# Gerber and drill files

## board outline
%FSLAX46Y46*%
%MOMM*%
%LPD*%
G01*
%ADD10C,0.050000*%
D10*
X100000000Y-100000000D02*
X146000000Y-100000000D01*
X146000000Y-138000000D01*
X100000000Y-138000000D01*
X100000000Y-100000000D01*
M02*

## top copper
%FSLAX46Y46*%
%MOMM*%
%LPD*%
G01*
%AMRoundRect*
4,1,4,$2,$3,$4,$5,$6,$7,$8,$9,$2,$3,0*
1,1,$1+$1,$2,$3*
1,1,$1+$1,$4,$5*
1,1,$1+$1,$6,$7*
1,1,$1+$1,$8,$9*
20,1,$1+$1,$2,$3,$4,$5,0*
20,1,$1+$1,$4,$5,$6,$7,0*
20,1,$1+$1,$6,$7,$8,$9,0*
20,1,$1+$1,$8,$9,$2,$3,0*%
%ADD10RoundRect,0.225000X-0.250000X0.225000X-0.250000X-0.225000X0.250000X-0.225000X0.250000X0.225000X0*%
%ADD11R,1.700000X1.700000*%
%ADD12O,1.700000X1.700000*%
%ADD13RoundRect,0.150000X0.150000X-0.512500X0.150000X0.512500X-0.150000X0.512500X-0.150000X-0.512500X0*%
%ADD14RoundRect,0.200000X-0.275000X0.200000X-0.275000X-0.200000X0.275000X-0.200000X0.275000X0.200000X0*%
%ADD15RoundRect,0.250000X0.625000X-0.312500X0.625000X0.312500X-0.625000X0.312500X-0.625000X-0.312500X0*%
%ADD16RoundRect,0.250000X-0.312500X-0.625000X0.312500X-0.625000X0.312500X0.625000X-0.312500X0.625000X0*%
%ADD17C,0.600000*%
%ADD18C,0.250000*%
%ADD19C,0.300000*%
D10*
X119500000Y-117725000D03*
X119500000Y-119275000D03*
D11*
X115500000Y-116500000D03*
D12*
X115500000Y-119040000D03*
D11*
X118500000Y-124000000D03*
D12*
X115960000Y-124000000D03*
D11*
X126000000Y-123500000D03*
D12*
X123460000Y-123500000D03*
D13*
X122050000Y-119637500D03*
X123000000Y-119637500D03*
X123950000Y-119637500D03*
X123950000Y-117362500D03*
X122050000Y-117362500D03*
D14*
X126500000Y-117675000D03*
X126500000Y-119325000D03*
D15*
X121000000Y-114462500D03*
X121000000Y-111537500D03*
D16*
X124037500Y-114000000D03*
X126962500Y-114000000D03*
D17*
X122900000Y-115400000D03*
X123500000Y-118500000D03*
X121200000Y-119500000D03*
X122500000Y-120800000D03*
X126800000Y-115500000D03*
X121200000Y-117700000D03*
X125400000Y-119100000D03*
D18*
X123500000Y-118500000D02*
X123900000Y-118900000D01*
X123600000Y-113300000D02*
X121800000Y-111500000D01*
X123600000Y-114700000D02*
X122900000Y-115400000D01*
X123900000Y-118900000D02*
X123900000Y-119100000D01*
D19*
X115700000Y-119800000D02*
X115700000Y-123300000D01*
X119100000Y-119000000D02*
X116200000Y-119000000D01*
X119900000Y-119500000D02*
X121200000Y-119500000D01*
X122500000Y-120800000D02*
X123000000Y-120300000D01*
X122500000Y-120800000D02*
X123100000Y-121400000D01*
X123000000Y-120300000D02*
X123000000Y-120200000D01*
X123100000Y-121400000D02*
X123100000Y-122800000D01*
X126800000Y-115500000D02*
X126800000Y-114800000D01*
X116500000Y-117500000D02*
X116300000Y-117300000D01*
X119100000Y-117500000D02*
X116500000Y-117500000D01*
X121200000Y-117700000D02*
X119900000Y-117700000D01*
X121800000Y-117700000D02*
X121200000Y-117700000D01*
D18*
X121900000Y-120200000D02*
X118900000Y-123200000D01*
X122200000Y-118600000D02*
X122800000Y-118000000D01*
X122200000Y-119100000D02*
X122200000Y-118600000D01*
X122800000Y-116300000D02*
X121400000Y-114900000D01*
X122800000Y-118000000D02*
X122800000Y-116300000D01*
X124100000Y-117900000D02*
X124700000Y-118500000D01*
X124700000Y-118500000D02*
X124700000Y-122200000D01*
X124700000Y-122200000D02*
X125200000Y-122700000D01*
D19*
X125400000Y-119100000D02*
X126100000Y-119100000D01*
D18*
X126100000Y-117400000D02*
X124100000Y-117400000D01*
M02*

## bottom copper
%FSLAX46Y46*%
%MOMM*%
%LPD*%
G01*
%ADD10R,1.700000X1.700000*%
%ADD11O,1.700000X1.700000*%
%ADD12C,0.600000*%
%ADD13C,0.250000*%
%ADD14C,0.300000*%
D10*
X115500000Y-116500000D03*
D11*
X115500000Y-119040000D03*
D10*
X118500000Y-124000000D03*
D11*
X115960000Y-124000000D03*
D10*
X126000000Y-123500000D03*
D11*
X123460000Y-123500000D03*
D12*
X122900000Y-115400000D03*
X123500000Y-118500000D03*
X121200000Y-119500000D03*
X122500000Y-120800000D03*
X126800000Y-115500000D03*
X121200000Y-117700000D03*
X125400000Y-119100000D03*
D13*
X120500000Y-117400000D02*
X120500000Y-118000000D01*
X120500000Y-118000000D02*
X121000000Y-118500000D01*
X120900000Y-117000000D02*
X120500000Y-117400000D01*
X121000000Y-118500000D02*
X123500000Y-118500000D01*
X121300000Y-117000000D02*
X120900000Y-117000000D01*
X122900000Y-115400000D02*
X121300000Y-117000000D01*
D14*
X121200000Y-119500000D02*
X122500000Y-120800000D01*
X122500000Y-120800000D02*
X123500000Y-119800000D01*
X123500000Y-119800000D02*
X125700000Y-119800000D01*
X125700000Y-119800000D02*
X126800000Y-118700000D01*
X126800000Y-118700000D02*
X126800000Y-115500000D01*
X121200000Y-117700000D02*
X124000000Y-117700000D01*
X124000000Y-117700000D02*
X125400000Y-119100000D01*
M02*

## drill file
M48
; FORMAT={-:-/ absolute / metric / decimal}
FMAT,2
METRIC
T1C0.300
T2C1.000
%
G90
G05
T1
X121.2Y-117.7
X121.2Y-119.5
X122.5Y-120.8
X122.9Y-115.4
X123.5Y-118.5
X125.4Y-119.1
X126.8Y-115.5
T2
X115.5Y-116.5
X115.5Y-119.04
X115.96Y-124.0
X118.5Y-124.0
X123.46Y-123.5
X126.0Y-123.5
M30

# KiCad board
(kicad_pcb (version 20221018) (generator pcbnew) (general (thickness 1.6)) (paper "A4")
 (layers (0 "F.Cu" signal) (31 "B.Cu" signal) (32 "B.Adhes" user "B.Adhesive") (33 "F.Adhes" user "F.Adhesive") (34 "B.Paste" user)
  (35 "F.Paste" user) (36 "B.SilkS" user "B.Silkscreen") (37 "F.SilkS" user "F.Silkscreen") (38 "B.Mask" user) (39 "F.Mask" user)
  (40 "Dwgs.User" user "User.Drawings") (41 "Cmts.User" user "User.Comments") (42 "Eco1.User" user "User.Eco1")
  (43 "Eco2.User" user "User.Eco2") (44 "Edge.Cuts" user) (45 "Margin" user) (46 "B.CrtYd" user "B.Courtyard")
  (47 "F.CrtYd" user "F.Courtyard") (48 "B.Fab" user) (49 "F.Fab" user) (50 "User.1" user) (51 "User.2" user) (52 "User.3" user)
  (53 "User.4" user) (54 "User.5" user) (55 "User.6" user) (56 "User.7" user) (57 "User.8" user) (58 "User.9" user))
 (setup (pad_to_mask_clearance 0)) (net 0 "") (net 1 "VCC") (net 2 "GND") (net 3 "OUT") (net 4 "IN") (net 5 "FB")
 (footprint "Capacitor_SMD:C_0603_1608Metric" (layer "F.Cu") (at 119.5 118.5 -90)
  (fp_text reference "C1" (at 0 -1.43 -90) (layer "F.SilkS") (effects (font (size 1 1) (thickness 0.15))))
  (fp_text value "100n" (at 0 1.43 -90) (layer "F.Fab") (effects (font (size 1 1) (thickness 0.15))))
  (pad "1" smd roundrect (at -0.775 0 270) (size 0.9 0.95) (layers "F.Cu" "F.Paste" "F.Mask") (roundrect_rratio 0.25) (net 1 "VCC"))
  (pad "2" smd roundrect (at 0.775 0 270) (size 0.9 0.95) (layers "F.Cu" "F.Paste" "F.Mask") (roundrect_rratio 0.25) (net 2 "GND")))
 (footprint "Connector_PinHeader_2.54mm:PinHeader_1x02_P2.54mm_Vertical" (layer "F.Cu") (at 115.5 116.5)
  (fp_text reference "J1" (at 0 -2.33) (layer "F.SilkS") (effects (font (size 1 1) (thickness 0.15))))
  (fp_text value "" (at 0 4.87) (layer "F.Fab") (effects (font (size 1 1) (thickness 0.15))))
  (pad "1" thru_hole rect (at 0 0) (size 1.7 1.7) (drill 1) (layers "*.Cu" "*.Mask") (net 1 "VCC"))
  (pad "2" thru_hole oval (at 0 2.54) (size 1.7 1.7) (drill 1) (layers "*.Cu" "*.Mask") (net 2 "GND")))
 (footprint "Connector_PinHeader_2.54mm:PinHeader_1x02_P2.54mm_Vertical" (layer "F.Cu") (at 118.5 124 -90)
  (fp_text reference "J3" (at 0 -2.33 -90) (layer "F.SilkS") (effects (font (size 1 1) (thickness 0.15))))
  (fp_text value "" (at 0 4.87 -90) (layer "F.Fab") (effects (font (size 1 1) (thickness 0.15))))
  (pad "1" thru_hole rect (at 0 0 270) (size 1.7 1.7) (drill 1) (layers "*.Cu" "*.Mask") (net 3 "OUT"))
  (pad "2" thru_hole oval (at 0 2.54 270) (size 1.7 1.7) (drill 1) (layers "*.Cu" "*.Mask") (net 2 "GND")))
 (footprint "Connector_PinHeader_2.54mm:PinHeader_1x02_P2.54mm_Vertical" (layer "F.Cu") (at 126 123.5 -90)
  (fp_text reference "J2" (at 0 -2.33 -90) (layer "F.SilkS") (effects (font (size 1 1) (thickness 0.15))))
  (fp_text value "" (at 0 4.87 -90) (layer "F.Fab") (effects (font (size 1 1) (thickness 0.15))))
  (pad "1" thru_hole rect (at 0 0 270) (size 1.7 1.7) (drill 1) (layers "*.Cu" "*.Mask") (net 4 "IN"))
  (pad "2" thru_hole oval (at 0 2.54 270) (size 1.7 1.7) (drill 1) (layers "*.Cu" "*.Mask") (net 2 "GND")))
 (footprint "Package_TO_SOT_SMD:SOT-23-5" (layer "F.Cu") (at 123 118.5 90)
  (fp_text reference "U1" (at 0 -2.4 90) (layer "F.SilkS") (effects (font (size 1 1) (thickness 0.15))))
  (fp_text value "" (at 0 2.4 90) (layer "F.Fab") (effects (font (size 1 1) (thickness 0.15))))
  (pad "1" smd roundrect (at -1.1375 -0.95 90) (size 1.325 0.6) (layers "F.Cu" "F.Paste" "F.Mask") (roundrect_rratio 0.25) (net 3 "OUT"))
  (pad "2" smd roundrect (at -1.1375 0 90) (size 1.325 0.6) (layers "F.Cu" "F.Paste" "F.Mask") (roundrect_rratio 0.25) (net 2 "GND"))
  (pad "3" smd roundrect (at -1.1375 0.95 90) (size 1.325 0.6) (layers "F.Cu" "F.Paste" "F.Mask") (roundrect_rratio 0.25) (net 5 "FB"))
  (pad "4" smd roundrect (at 1.1375 0.95 90) (size 1.325 0.6) (layers "F.Cu" "F.Paste" "F.Mask") (roundrect_rratio 0.25) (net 4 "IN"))
  (pad "5" smd roundrect (at 1.1375 -0.95 90) (size 1.325 0.6) (layers "F.Cu" "F.Paste" "F.Mask") (roundrect_rratio 0.25) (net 1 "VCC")))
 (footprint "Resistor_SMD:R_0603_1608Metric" (layer "F.Cu") (at 126.5 118.5 -90)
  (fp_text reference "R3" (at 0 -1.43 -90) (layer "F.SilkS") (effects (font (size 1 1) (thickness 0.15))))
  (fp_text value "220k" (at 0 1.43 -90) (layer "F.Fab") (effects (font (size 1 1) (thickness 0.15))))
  (pad "1" smd roundrect (at -0.825 0 270) (size 0.8 0.95) (layers "F.Cu" "F.Paste" "F.Mask") (roundrect_rratio 0.25) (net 4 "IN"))
  (pad "2" smd roundrect (at 0.825 0 270) (size 0.8 0.95) (layers "F.Cu" "F.Paste" "F.Mask") (roundrect_rratio 0.25) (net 1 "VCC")))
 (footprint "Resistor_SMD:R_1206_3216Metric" (layer "F.Cu") (at 121 113 90)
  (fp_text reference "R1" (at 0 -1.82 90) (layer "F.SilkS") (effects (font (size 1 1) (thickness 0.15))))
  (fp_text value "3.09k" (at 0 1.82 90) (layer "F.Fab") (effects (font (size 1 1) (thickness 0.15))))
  (pad "1" smd roundrect (at -1.4625 0 90) (size 1.125 1.75) (layers "F.Cu" "F.Paste" "F.Mask") (roundrect_rratio 0.222222) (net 3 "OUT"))
  (pad "2" smd roundrect (at 1.4625 0 90) (size 1.125 1.75) (layers "F.Cu" "F.Paste" "F.Mask") (roundrect_rratio 0.222222) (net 5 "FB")))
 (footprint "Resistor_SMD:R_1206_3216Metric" (layer "F.Cu") (at 125.5 114)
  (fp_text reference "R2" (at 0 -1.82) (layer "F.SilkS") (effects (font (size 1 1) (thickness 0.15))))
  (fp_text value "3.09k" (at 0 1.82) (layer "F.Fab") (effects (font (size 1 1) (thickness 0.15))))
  (pad "1" smd roundrect (at -1.4625 0) (size 1.125 1.75) (layers "F.Cu" "F.Paste" "F.Mask") (roundrect_rratio 0.222222) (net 5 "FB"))
  (pad "2" smd roundrect (at 1.4625 0) (size 1.125 1.75) (layers "F.Cu" "F.Paste" "F.Mask") (roundrect_rratio 0.222222) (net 2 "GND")))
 (gr_rect (start 100 100) (end 146 138) (stroke (width 0.05) (type default)) (fill none) (layer "Edge.Cuts"))
 (segment (start 123.5 118.5) (end 123.9 118.9) (width 0.25) (layer "F.Cu") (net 5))
 (segment (start 123.6 113.3) (end 121.8 111.5) (width 0.25) (layer "F.Cu") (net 5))
 (segment (start 123.6 114.7) (end 122.9 115.4) (width 0.25) (layer "F.Cu") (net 5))
 (segment (start 123.9 118.9) (end 123.9 119.1) (width 0.25) (layer "F.Cu") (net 5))
 (via (at 122.9 115.4) (size 0.6) (drill 0.3) (layers "F.Cu" "B.Cu") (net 5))
 (via (at 123.5 118.5) (size 0.6) (drill 0.3) (layers "F.Cu" "B.Cu") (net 5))
 (segment (start 115.7 119.8) (end 115.7 123.3) (width 0.3) (layer "F.Cu") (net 2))
 (segment (start 119.1 119) (end 116.2 119) (width 0.3) (layer "F.Cu") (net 2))
 (segment (start 119.9 119.5) (end 121.2 119.5) (width 0.3) (layer "F.Cu") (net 2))
 (segment (start 120.5 117.4) (end 120.5 118) (width 0.25) (layer "B.Cu") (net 5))
 (segment (start 120.5 118) (end 121 118.5) (width 0.25) (layer "B.Cu") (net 5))
 (segment (start 120.9 117) (end 120.5 117.4) (width 0.25) (layer "B.Cu") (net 5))
 (segment (start 121 118.5) (end 123.5 118.5) (width 0.25) (layer "B.Cu") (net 5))
 (segment (start 121.3 117) (end 120.9 117) (width 0.25) (layer "B.Cu") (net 5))
 (segment (start 122.5 120.8) (end 123 120.3) (width 0.3) (layer "F.Cu") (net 2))
 (segment (start 122.5 120.8) (end 123.1 121.4) (width 0.3) (layer "F.Cu") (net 2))
 (segment (start 122.9 115.4) (end 121.3 117) (width 0.25) (layer "B.Cu") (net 5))
 (segment (start 123 120.3) (end 123 120.2) (width 0.3) (layer "F.Cu") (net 2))
 (segment (start 123.1 121.4) (end 123.1 122.8) (width 0.3) (layer "F.Cu") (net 2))
 (segment (start 126.8 115.5) (end 126.8 114.8) (width 0.3) (layer "F.Cu") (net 2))
 (via (at 121.2 119.5) (size 0.6) (drill 0.3) (layers "F.Cu" "B.Cu") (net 2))
 (via (at 122.5 120.8) (size 0.6) (drill 0.3) (layers "F.Cu" "B.Cu") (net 2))
 (via (at 126.8 115.5) (size 0.6) (drill 0.3) (layers "F.Cu" "B.Cu") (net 2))
 (segment (start 116.5 117.5) (end 116.3 117.3) (width 0.3) (layer "F.Cu") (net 1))
 (segment (start 119.1 117.5) (end 116.5 117.5) (width 0.3) (layer "F.Cu") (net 1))
 (segment (start 121.2 117.7) (end 119.9 117.7) (width 0.3) (layer "F.Cu") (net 1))
 (segment (start 121.2 119.5) (end 122.5 120.8) (width 0.3) (layer "B.Cu") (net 2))
 (segment (start 121.8 117.7) (end 121.2 117.7) (width 0.3) (layer "F.Cu") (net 1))
 (segment (start 121.9 120.2) (end 118.9 123.2) (width 0.25) (layer "F.Cu") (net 3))
 (segment (start 122.2 118.6) (end 122.8 118) (width 0.25) (layer "F.Cu") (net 3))
 (segment (start 122.2 119.1) (end 122.2 118.6) (width 0.25) (layer "F.Cu") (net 3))
 (segment (start 122.5 120.8) (end 123.5 119.8) (width 0.3) (layer "B.Cu") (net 2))
 (segment (start 122.8 116.3) (end 121.4 114.9) (width 0.25) (layer "F.Cu") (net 3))
 (segment (start 122.8 118) (end 122.8 116.3) (width 0.25) (layer "F.Cu") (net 3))
 (segment (start 123.5 119.8) (end 125.7 119.8) (width 0.3) (layer "B.Cu") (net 2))
 (segment (start 124.1 117.9) (end 124.7 118.5) (width 0.25) (layer "F.Cu") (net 4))
 (segment (start 124.7 118.5) (end 124.7 122.2) (width 0.25) (layer "F.Cu") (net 4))
 (segment (start 124.7 122.2) (end 125.2 122.7) (width 0.25) (layer "F.Cu") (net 4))
 (segment (start 125.4 119.1) (end 126.1 119.1) (width 0.3) (layer "F.Cu") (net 1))
 (segment (start 125.7 119.8) (end 126.8 118.7) (width 0.3) (layer "B.Cu") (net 2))
 (segment (start 126.1 117.4) (end 124.1 117.4) (width 0.25) (layer "F.Cu") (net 4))
 (segment (start 126.8 118.7) (end 126.8 115.5) (width 0.3) (layer "B.Cu") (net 2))
 (via (at 121.2 117.7) (size 0.6) (drill 0.3) (layers "F.Cu" "B.Cu") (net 1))
 (via (at 125.4 119.1) (size 0.6) (drill 0.3) (layers "F.Cu" "B.Cu") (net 1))
 (segment (start 121.2 117.7) (end 124 117.7) (width 0.3) (layer "B.Cu") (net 1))
 (segment (start 124 117.7) (end 125.4 119.1) (width 0.3) (layer "B.Cu") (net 1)))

